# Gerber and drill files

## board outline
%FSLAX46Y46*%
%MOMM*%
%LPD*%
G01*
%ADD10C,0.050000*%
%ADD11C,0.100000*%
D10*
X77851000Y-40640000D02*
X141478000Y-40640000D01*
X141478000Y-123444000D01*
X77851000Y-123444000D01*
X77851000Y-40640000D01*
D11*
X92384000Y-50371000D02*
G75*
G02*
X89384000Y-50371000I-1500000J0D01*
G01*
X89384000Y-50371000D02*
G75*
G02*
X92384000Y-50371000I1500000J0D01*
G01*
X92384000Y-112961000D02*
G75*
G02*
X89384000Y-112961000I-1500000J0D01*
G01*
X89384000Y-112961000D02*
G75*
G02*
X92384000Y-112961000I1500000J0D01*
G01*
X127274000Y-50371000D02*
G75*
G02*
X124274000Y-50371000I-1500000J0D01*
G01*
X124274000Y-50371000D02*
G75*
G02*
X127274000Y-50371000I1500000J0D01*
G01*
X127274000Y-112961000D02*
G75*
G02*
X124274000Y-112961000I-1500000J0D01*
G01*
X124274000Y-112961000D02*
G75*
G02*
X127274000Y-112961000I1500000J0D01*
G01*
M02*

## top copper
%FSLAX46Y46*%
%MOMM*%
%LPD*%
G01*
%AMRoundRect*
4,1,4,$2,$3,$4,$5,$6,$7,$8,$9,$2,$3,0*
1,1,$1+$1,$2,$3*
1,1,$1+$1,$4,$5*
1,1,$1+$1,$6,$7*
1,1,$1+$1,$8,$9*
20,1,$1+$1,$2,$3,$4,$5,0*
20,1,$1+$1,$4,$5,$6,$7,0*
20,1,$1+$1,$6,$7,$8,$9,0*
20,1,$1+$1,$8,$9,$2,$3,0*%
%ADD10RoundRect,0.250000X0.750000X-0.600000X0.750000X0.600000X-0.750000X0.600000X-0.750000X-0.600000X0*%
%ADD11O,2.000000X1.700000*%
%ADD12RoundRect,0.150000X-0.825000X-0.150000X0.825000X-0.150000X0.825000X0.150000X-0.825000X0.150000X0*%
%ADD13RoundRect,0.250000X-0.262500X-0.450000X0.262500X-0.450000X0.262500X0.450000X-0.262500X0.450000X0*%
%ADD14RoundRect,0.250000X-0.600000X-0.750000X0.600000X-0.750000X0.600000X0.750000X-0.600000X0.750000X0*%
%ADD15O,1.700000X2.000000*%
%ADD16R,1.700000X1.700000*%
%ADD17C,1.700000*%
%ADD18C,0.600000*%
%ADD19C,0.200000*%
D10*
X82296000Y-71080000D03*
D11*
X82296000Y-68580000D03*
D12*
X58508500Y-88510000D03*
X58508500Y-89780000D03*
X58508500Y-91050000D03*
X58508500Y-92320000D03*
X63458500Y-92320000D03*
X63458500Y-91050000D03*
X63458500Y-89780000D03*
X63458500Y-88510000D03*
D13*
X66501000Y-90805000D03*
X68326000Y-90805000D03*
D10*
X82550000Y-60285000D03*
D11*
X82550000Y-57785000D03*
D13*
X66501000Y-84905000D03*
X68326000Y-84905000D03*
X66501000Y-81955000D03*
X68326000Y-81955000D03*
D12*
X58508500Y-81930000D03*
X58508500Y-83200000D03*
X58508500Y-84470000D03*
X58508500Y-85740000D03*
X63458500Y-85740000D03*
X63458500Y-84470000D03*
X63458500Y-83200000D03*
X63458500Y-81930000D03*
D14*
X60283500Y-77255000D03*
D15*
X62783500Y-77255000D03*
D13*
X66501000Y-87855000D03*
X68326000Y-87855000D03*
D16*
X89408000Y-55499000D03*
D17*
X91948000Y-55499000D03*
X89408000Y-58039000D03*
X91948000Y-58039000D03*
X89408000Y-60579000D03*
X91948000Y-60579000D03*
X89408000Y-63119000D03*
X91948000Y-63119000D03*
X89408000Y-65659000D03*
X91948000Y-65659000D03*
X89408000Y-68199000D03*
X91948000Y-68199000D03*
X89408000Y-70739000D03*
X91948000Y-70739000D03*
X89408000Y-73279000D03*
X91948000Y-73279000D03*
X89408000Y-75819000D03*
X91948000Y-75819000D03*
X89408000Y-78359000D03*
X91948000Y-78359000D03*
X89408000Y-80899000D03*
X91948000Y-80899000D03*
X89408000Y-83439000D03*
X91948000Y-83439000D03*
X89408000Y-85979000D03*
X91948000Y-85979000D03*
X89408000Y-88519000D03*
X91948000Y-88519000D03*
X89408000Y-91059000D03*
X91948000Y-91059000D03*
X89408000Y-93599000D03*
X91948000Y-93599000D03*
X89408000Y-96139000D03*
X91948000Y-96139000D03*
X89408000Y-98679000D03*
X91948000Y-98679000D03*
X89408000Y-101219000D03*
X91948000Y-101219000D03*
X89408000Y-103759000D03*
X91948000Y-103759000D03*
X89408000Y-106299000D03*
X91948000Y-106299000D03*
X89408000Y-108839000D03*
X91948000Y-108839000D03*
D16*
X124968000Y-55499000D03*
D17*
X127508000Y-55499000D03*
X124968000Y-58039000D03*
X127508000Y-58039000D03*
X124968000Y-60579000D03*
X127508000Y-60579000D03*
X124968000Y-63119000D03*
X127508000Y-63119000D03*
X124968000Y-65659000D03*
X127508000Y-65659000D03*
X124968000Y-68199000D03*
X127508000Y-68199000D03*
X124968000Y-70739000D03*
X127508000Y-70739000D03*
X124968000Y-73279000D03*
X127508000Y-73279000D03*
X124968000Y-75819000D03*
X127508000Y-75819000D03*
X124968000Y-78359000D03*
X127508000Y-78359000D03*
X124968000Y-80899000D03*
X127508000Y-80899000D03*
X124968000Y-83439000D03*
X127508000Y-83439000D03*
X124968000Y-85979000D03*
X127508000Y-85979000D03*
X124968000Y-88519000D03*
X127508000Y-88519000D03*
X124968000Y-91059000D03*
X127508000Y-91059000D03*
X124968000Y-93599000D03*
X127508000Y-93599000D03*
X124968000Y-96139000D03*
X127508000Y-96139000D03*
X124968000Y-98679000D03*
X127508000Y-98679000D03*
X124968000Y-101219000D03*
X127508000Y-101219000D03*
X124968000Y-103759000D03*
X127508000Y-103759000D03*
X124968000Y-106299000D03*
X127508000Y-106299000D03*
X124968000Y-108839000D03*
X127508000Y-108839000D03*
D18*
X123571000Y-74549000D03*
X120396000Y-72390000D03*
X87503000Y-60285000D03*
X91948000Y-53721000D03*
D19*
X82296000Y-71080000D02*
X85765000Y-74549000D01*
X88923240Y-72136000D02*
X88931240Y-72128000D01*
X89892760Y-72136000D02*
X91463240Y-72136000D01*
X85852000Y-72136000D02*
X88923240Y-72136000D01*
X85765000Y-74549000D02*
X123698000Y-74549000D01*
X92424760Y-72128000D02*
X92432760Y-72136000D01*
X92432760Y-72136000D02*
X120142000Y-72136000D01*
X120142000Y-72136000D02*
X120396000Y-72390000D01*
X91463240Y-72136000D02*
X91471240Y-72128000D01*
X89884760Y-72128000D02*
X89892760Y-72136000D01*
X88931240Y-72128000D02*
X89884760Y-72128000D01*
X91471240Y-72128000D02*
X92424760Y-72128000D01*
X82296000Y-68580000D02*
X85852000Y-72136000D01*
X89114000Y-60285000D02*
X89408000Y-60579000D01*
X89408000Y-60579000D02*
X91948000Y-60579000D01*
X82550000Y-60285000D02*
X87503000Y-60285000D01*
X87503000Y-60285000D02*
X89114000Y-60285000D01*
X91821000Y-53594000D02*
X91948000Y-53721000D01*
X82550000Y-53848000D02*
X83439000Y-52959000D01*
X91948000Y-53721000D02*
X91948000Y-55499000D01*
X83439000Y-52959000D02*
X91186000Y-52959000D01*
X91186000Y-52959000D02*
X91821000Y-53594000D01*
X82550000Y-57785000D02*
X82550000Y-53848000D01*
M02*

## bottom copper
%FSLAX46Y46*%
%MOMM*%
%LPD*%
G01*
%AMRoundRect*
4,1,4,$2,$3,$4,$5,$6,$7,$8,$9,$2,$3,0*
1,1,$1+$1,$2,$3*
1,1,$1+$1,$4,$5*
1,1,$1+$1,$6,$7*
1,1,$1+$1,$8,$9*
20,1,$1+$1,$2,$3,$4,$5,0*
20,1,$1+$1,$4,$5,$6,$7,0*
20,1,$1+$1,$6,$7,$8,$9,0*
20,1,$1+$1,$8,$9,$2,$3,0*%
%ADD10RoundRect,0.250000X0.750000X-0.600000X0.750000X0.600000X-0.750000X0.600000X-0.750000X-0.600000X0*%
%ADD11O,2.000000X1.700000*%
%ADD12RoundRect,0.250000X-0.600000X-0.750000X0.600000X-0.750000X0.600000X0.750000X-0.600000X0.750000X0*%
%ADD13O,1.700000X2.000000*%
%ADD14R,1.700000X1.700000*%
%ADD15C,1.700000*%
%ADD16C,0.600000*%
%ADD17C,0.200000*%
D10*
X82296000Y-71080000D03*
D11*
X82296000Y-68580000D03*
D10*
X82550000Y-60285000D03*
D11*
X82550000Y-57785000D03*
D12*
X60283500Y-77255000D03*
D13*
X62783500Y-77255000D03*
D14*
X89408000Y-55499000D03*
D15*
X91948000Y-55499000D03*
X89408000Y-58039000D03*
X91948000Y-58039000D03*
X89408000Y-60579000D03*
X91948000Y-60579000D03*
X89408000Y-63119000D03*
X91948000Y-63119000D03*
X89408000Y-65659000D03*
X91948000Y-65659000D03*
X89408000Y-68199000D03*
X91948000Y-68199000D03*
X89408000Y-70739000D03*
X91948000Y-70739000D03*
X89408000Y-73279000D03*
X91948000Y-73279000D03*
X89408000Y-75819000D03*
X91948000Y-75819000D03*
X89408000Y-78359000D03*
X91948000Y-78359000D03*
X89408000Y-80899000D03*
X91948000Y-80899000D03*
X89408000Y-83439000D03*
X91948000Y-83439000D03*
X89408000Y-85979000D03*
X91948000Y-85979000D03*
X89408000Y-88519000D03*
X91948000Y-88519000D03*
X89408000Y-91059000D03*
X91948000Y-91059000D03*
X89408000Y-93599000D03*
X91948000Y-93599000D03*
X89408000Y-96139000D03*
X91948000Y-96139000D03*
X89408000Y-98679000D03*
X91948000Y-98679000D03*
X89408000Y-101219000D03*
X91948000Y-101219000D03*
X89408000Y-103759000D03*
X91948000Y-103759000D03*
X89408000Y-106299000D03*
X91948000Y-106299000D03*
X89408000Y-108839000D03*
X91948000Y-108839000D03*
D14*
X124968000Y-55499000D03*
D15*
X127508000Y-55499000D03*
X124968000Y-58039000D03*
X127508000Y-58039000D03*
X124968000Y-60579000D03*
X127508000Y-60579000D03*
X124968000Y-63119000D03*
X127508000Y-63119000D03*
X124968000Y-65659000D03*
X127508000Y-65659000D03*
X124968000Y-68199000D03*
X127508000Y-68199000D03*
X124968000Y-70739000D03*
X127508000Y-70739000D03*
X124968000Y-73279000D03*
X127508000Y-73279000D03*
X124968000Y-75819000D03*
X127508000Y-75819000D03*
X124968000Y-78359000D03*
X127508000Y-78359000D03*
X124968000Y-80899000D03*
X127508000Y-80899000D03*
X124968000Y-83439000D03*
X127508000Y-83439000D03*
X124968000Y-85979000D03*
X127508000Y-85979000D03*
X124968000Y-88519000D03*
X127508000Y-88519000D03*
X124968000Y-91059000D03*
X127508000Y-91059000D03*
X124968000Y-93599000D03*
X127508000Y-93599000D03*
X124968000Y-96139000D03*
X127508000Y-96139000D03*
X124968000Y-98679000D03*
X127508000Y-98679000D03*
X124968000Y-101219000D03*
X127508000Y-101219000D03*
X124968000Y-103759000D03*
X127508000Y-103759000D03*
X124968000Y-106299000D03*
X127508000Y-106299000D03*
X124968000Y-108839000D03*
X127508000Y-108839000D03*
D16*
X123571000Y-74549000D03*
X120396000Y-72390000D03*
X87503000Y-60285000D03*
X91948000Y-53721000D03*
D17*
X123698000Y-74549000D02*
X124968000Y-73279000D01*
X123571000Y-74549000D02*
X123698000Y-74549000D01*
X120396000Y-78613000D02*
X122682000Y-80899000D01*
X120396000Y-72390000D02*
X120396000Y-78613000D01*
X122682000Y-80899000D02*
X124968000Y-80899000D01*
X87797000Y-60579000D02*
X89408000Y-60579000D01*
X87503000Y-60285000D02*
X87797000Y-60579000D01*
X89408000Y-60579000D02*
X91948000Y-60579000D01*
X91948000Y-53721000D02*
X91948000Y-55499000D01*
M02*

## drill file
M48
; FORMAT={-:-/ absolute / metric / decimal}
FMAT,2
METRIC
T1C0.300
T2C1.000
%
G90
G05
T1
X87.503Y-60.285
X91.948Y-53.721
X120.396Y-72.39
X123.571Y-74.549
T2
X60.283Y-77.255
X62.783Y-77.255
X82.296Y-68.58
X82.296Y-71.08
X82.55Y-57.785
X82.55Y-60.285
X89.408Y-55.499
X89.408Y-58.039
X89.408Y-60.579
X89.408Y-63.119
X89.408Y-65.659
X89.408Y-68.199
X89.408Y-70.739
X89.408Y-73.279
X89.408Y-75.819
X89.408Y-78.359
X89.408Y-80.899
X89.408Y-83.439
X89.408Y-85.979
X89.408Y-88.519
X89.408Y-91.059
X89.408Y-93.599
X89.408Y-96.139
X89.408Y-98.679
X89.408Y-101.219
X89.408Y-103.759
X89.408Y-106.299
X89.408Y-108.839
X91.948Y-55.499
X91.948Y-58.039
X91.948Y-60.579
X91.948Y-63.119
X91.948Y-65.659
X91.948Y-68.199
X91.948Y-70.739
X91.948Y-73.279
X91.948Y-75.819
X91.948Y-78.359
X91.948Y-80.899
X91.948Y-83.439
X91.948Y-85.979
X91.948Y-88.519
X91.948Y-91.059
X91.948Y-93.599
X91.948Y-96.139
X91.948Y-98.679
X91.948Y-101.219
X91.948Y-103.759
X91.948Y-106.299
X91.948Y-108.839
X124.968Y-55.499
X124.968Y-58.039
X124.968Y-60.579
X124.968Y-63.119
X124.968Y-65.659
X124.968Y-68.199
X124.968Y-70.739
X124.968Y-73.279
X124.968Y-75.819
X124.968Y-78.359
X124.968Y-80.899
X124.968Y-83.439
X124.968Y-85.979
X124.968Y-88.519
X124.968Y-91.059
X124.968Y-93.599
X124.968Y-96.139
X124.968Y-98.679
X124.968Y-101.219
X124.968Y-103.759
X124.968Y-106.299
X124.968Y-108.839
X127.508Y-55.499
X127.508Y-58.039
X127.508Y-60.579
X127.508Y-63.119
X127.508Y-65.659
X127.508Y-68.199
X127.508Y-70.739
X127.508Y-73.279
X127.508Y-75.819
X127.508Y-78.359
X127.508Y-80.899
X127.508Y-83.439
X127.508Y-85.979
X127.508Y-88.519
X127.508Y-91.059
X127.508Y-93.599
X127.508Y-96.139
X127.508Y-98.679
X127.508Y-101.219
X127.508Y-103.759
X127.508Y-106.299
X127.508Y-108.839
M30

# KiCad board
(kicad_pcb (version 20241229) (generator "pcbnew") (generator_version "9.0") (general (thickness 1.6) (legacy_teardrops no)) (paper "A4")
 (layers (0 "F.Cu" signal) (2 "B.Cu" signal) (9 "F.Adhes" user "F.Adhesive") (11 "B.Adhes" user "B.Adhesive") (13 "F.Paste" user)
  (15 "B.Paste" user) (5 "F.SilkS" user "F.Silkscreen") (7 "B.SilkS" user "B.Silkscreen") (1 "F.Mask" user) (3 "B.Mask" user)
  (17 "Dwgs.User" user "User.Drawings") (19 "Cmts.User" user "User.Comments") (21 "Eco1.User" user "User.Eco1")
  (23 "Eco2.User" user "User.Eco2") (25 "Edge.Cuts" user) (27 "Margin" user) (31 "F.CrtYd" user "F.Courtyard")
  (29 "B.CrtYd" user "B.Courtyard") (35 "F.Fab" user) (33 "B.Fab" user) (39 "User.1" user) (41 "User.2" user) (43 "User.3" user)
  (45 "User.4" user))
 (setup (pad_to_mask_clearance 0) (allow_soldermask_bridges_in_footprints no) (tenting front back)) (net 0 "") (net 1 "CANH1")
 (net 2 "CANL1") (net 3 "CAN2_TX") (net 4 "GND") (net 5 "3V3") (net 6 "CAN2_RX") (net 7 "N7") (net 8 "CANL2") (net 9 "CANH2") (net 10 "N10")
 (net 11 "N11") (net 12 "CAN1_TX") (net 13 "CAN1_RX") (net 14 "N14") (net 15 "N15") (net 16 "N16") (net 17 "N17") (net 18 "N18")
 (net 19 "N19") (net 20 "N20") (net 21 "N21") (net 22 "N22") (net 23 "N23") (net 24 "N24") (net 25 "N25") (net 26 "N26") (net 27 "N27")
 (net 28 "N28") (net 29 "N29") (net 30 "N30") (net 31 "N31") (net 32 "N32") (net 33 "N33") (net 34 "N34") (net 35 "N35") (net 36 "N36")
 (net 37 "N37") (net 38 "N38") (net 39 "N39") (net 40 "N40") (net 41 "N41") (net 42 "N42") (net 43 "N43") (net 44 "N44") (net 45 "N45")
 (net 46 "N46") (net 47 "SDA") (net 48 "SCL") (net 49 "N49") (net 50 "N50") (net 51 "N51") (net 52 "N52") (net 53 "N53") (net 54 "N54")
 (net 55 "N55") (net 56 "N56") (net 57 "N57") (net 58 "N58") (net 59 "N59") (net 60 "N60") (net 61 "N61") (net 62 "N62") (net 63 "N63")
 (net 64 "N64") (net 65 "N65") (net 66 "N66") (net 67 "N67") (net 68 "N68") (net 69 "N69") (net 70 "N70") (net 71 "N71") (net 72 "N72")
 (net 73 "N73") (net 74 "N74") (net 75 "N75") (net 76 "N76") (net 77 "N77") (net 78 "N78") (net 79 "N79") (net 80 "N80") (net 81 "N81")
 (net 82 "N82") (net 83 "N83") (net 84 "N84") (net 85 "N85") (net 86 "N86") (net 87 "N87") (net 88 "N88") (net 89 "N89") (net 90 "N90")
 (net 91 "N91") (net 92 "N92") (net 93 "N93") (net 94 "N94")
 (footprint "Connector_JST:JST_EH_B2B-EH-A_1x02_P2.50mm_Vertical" (layer "F.Cu") (at 82.296 71.08 90)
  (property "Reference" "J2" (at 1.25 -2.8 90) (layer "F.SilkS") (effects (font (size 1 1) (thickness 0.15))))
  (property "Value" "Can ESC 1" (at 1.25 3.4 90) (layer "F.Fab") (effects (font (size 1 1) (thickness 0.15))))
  (pad "1" thru_hole roundrect (at 0 0 90) (size 1.7 2) (drill 1) (layers "*.Cu" "*.Mask") (remove_unused_layers no)
   (roundrect_rratio 0.147059) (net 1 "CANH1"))
  (pad "2" thru_hole oval (at 2.5 0 90) (size 1.7 2) (drill 1) (layers "*.Cu" "*.Mask") (remove_unused_layers no) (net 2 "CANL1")))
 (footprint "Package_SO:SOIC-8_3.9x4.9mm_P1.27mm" (layer "F.Cu") (at 60.9835 90.415)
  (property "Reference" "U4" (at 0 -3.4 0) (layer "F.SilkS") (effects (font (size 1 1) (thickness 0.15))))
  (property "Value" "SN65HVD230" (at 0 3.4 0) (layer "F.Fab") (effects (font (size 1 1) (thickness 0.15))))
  (pad "1" smd roundrect (at -2.475 -1.905) (size 1.95 0.6) (layers "F.Cu" "F.Mask" "F.Paste") (roundrect_rratio 0.25) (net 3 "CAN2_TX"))
  (pad "2" smd roundrect (at -2.475 -0.635) (size 1.95 0.6) (layers "F.Cu" "F.Mask" "F.Paste") (roundrect_rratio 0.25) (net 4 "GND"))
  (pad "3" smd roundrect (at -2.475 0.635) (size 1.95 0.6) (layers "F.Cu" "F.Mask" "F.Paste") (roundrect_rratio 0.25) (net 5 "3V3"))
  (pad "4" smd roundrect (at -2.475 1.905) (size 1.95 0.6) (layers "F.Cu" "F.Mask" "F.Paste") (roundrect_rratio 0.25) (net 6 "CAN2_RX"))
  (pad "5" smd roundrect (at 2.475 1.905) (size 1.95 0.6) (layers "F.Cu" "F.Mask" "F.Paste") (roundrect_rratio 0.25) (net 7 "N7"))
  (pad "6" smd roundrect (at 2.475 0.635) (size 1.95 0.6) (layers "F.Cu" "F.Mask" "F.Paste") (roundrect_rratio 0.25) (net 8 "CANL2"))
  (pad "7" smd roundrect (at 2.475 -0.635) (size 1.95 0.6) (layers "F.Cu" "F.Mask" "F.Paste") (roundrect_rratio 0.25) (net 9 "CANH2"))
  (pad "8" smd roundrect (at 2.475 -1.905) (size 1.95 0.6) (layers "F.Cu" "F.Mask" "F.Paste") (roundrect_rratio 0.25) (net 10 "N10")))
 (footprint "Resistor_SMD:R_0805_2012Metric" (layer "F.Cu") (at 67.4135 90.805)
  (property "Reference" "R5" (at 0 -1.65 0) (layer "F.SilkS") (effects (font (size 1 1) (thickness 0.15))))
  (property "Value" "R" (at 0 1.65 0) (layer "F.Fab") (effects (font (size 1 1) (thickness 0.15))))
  (pad "1" smd roundrect (at -0.9125 0) (size 1.025 1.4) (layers "F.Cu" "F.Mask" "F.Paste") (roundrect_rratio 0.243902) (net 4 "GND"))
  (pad "2" smd roundrect (at 0.9125 0) (size 1.025 1.4) (layers "F.Cu" "F.Mask" "F.Paste") (roundrect_rratio 0.243902) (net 10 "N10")))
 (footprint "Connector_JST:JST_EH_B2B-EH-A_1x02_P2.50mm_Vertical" (layer "F.Cu") (at 82.55 60.285 90)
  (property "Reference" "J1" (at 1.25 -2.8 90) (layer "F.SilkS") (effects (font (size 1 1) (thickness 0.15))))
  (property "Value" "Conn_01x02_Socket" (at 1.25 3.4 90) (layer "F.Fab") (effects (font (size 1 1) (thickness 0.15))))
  (pad "1" thru_hole roundrect (at 0 0 90) (size 1.7 2) (drill 1) (layers "*.Cu" "*.Mask") (remove_unused_layers no)
   (roundrect_rratio 0.147059) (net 4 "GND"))
  (pad "2" thru_hole oval (at 2.5 0 90) (size 1.7 2) (drill 1) (layers "*.Cu" "*.Mask") (remove_unused_layers no) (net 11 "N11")))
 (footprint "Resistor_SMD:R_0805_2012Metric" (layer "F.Cu") (at 67.4135 84.905)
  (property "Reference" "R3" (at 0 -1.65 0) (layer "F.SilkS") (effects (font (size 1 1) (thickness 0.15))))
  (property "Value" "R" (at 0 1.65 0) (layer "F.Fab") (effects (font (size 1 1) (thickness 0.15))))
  (pad "1" smd roundrect (at -0.9125 0) (size 1.025 1.4) (layers "F.Cu" "F.Mask" "F.Paste") (roundrect_rratio 0.243902) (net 9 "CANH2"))
  (pad "2" smd roundrect (at 0.9125 0) (size 1.025 1.4) (layers "F.Cu" "F.Mask" "F.Paste") (roundrect_rratio 0.243902) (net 8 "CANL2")))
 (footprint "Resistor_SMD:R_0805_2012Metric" (layer "F.Cu") (at 67.4135 81.955)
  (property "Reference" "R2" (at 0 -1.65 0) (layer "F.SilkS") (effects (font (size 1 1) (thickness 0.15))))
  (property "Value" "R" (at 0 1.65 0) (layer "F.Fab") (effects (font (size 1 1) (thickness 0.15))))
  (pad "1" smd roundrect (at -0.9125 0) (size 1.025 1.4) (layers "F.Cu" "F.Mask" "F.Paste") (roundrect_rratio 0.243902) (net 1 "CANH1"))
  (pad "2" smd roundrect (at 0.9125 0) (size 1.025 1.4) (layers "F.Cu" "F.Mask" "F.Paste") (roundrect_rratio 0.243902) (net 2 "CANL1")))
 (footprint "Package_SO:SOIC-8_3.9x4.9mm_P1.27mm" (layer "F.Cu") (at 60.9835 83.835)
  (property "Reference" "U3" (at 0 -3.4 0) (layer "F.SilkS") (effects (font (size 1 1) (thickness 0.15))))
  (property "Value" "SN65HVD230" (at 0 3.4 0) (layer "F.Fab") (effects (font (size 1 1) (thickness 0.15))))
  (pad "1" smd roundrect (at -2.475 -1.905) (size 1.95 0.6) (layers "F.Cu" "F.Mask" "F.Paste") (roundrect_rratio 0.25) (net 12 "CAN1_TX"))
  (pad "2" smd roundrect (at -2.475 -0.635) (size 1.95 0.6) (layers "F.Cu" "F.Mask" "F.Paste") (roundrect_rratio 0.25) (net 4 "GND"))
  (pad "3" smd roundrect (at -2.475 0.635) (size 1.95 0.6) (layers "F.Cu" "F.Mask" "F.Paste") (roundrect_rratio 0.25) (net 5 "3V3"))
  (pad "4" smd roundrect (at -2.475 1.905) (size 1.95 0.6) (layers "F.Cu" "F.Mask" "F.Paste") (roundrect_rratio 0.25) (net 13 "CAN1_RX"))
  (pad "5" smd roundrect (at 2.475 1.905) (size 1.95 0.6) (layers "F.Cu" "F.Mask" "F.Paste") (roundrect_rratio 0.25) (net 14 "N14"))
  (pad "6" smd roundrect (at 2.475 0.635) (size 1.95 0.6) (layers "F.Cu" "F.Mask" "F.Paste") (roundrect_rratio 0.25) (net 2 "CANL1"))
  (pad "7" smd roundrect (at 2.475 -0.635) (size 1.95 0.6) (layers "F.Cu" "F.Mask" "F.Paste") (roundrect_rratio 0.25) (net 1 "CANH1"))
  (pad "8" smd roundrect (at 2.475 -1.905) (size 1.95 0.6) (layers "F.Cu" "F.Mask" "F.Paste") (roundrect_rratio 0.25) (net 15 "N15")))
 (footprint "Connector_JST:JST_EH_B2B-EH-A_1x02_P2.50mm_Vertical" (layer "F.Cu") (at 60.2835 77.255)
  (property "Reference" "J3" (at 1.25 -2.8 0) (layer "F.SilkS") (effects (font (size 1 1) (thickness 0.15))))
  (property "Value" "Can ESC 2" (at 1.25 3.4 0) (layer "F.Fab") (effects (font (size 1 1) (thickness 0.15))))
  (pad "1" thru_hole roundrect (at 0 0) (size 1.7 2) (drill 1) (layers "*.Cu" "*.Mask") (remove_unused_layers no)
   (roundrect_rratio 0.147059) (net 9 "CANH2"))
  (pad "2" thru_hole oval (at 2.5 0) (size 1.7 2) (drill 1) (layers "*.Cu" "*.Mask") (remove_unused_layers no) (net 8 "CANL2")))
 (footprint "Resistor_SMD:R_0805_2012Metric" (layer "F.Cu") (at 67.4135 87.855)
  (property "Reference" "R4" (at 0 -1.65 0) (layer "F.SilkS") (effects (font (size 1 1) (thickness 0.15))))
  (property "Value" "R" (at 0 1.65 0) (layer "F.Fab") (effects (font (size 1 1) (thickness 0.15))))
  (pad "1" smd roundrect (at -0.9125 0) (size 1.025 1.4) (layers "F.Cu" "F.Mask" "F.Paste") (roundrect_rratio 0.243902) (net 4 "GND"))
  (pad "2" smd roundrect (at 0.9125 0) (size 1.025 1.4) (layers "F.Cu" "F.Mask" "F.Paste") (roundrect_rratio 0.243902) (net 15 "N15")))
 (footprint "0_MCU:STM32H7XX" (layer "F.Cu") (at 99.568 38.735)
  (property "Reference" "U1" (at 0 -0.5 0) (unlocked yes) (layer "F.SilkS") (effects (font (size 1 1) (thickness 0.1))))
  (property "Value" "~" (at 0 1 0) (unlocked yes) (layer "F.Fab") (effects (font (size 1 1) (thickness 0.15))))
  (fp_circle (center -8.684 11.636) (end -7.184 11.636) (stroke (width 0.1) (type solid)) (fill no) (layer "Edge.Cuts"))
  (fp_circle (center -8.684 74.226) (end -7.184 74.226) (stroke (width 0.1) (type solid)) (fill no) (layer "Edge.Cuts"))
  (fp_circle (center 26.206 11.636) (end 27.706 11.636) (stroke (width 0.1) (type solid)) (fill no) (layer "Edge.Cuts"))
  (fp_circle (center 26.206 74.226) (end 27.706 74.226) (stroke (width 0.1) (type solid)) (fill no) (layer "Edge.Cuts"))
  (pad "1" thru_hole rect (at -10.16 16.764 180) (size 1.7 1.7) (drill 1) (layers "*.Cu" "*.Mask") (remove_unused_layers no) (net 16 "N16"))
  (pad "2" thru_hole circle (at -7.62 16.764 180) (size 1.7 1.7) (drill 1) (layers "*.Cu" "*.Mask") (remove_unused_layers no) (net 11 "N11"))
  (pad "3" thru_hole circle (at -10.16 19.304 180) (size 1.7 1.7) (drill 1) (layers "*.Cu" "*.Mask") (remove_unused_layers no) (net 5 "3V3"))
  (pad "4" thru_hole circle (at -7.62 19.304 180) (size 1.7 1.7) (drill 1) (layers "*.Cu" "*.Mask") (remove_unused_layers no) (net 5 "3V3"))
  (pad "5" thru_hole circle (at -10.16 21.844 180) (size 1.7 1.7) (drill 1) (layers "*.Cu" "*.Mask") (remove_unused_layers no) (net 4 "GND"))
  (pad "6" thru_hole circle (at -7.62 21.844 180) (size 1.7 1.7) (drill 1) (layers "*.Cu" "*.Mask") (remove_unused_layers no) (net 4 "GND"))
  (pad "7" thru_hole circle (at -10.16 24.384 180) (size 1.7 1.7) (drill 1) (layers "*.Cu" "*.Mask") (remove_unused_layers no)
   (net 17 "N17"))
  (pad "8" thru_hole circle (at -7.62 24.384 180) (size 1.7 1.7) (drill 1) (layers "*.Cu" "*.Mask") (remove_unused_layers no) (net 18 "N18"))
  (pad "9" thru_hole circle (at -10.16 26.924 180) (size 1.7 1.7) (drill 1) (layers "*.Cu" "*.Mask") (remove_unused_layers no)
   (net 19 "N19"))
  (pad "10" thru_hole circle (at -7.62 26.924 180) (size 1.7 1.7) (drill 1) (layers "*.Cu" "*.Mask") (remove_unused_layers no)
   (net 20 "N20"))
  (pad "11" thru_hole circle (at -10.16 29.464 180) (size 1.7 1.7) (drill 1) (layers "*.Cu" "*.Mask") (remove_unused_layers no)
   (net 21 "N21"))
  (pad "12" thru_hole circle (at -7.62 29.464 180) (size 1.7 1.7) (drill 1) (layers "*.Cu" "*.Mask") (remove_unused_layers no)
   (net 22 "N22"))
  (pad "13" thru_hole circle (at -10.16 32.004 180) (size 1.7 1.7) (drill 1) (layers "*.Cu" "*.Mask") (remove_unused_layers no)
   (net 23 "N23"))
  (pad "14" thru_hole circle (at -7.62 32.004 180) (size 1.7 1.7) (drill 1) (layers "*.Cu" "*.Mask") (remove_unused_layers no)
   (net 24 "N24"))
  (pad "15" thru_hole circle (at -10.16 34.544 180) (size 1.7 1.7) (drill 1) (layers "*.Cu" "*.Mask") (remove_unused_layers no)
   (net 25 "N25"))
  (pad "16" thru_hole circle (at -7.62 34.544 180) (size 1.7 1.7) (drill 1) (layers "*.Cu" "*.Mask") (remove_unused_layers no)
   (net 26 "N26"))
  (pad "17" thru_hole circle (at -10.16 37.084 180) (size 1.7 1.7) (drill 1) (layers "*.Cu" "*.Mask") (remove_unused_layers no)
   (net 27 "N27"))
  (pad "18" thru_hole circle (at -7.62 37.084 180) (size 1.7 1.7) (drill 1) (layers "*.Cu" "*.Mask") (remove_unused_layers no)
   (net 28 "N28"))
  (pad "19" thru_hole circle (at -10.16 39.624 180) (size 1.7 1.7) (drill 1) (layers "*.Cu" "*.Mask") (remove_unused_layers no)
   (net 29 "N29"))
  (pad "20" thru_hole circle (at -7.62 39.624 180) (size 1.7 1.7) (drill 1) (layers "*.Cu" "*.Mask") (remove_unused_layers no)
   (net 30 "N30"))
  (pad "21" thru_hole circle (at -10.16 42.164 180) (size 1.7 1.7) (drill 1) (layers "*.Cu" "*.Mask") (remove_unused_layers no)
   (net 12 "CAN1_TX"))
  (pad "22" thru_hole circle (at -7.62 42.164 180) (size 1.7 1.7) (drill 1) (layers "*.Cu" "*.Mask") (remove_unused_layers no)
   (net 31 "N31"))
  (pad "23" thru_hole circle (at -10.16 44.704 180) (size 1.7 1.7) (drill 1) (layers "*.Cu" "*.Mask") (remove_unused_layers no)
   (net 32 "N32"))
  (pad "24" thru_hole circle (at -7.62 44.704 180) (size 1.7 1.7) (drill 1) (layers "*.Cu" "*.Mask") (remove_unused_layers no)
   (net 13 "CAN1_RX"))
  (pad "25" thru_hole circle (at -10.16 47.244 180) (size 1.7 1.7) (drill 1) (layers "*.Cu" "*.Mask") (remove_unused_layers no)
   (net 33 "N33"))
  (pad "26" thru_hole circle (at -7.62 47.244 180) (size 1.7 1.7) (drill 1) (layers "*.Cu" "*.Mask") (remove_unused_layers no)
   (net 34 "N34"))
  (pad "27" thru_hole circle (at -10.16 49.784 180) (size 1.7 1.7) (drill 1) (layers "*.Cu" "*.Mask") (remove_unused_layers no)
   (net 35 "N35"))
  (pad "28" thru_hole circle (at -7.62 49.784 180) (size 1.7 1.7) (drill 1) (layers "*.Cu" "*.Mask") (remove_unused_layers no)
   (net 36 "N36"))
  (pad "29" thru_hole circle (at -10.16 52.324 180) (size 1.7 1.7) (drill 1) (layers "*.Cu" "*.Mask") (remove_unused_layers no)
   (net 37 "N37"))
  (pad "30" thru_hole circle (at -7.62 52.324 180) (size 1.7 1.7) (drill 1) (layers "*.Cu" "*.Mask") (remove_unused_layers no)
   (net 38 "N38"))
  (pad "31" thru_hole circle (at -10.16 54.864 180) (size 1.7 1.7) (drill 1) (layers "*.Cu" "*.Mask") (remove_unused_layers no)
   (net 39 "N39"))
  (pad "32" thru_hole circle (at -7.62 54.864 180) (size 1.7 1.7) (drill 1) (layers "*.Cu" "*.Mask") (remove_unused_layers no)
   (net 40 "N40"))
  (pad "33" thru_hole circle (at -10.16 57.404 180) (size 1.7 1.7) (drill 1) (layers "*.Cu" "*.Mask") (remove_unused_layers no)
   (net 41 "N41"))
  (pad "34" thru_hole circle (at -7.62 57.404 180) (size 1.7 1.7) (drill 1) (layers "*.Cu" "*.Mask") (remove_unused_layers no)
   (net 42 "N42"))
  (pad "35" thru_hole circle (at -10.16 59.944 180) (size 1.7 1.7) (drill 1) (layers "*.Cu" "*.Mask") (remove_unused_layers no)
   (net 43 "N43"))
  (pad "36" thru_hole circle (at -7.62 59.944 180) (size 1.7 1.7) (drill 1) (layers "*.Cu" "*.Mask") (remove_unused_layers no)
   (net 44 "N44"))
  (pad "37" thru_hole circle (at -10.16 62.484 180) (size 1.7 1.7) (drill 1) (layers "*.Cu" "*.Mask") (remove_unused_layers no)
   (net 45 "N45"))
  (pad "38" thru_hole circle (at -7.62 62.484 180) (size 1.7 1.7) (drill 1) (layers "*.Cu" "*.Mask") (remove_unused_layers no)
   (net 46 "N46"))
  (pad "39" thru_hole circle (at -10.16 65.024 180) (size 1.7 1.7) (drill 1) (layers "*.Cu" "*.Mask") (remove_unused_layers no)
   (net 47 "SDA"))
  (pad "40" thru_hole circle (at -7.62 65.024 180) (size 1.7 1.7) (drill 1) (layers "*.Cu" "*.Mask") (remove_unused_layers no)
   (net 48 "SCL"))
  (pad "41" thru_hole circle (at -10.16 67.564 180) (size 1.7 1.7) (drill 1) (layers "*.Cu" "*.Mask") (remove_unused_layers no)
   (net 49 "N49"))
  (pad "42" thru_hole circle (at -7.62 67.564 180) (size 1.7 1.7) (drill 1) (layers "*.Cu" "*.Mask") (remove_unused_layers no)
   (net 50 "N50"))
  (pad "43" thru_hole circle (at -10.16 70.104 180) (size 1.7 1.7) (drill 1) (layers "*.Cu" "*.Mask") (remove_unused_layers no)
   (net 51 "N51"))
  (pad "44" thru_hole circle (at -7.62 70.104 180) (size 1.7 1.7) (drill 1) (layers "*.Cu" "*.Mask") (remove_unused_layers no)
   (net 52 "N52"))
  (pad "45" thru_hole rect (at 25.4 16.764 180) (size 1.7 1.7) (drill 1) (layers "*.Cu" "*.Mask") (remove_unused_layers no) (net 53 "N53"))
  (pad "46" thru_hole circle (at 27.94 16.764 180) (size 1.7 1.7) (drill 1) (layers "*.Cu" "*.Mask") (remove_unused_layers no)
   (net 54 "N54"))
  (pad "47" thru_hole circle (at 25.4 19.304 180) (size 1.7 1.7) (drill 1) (layers "*.Cu" "*.Mask") (remove_unused_layers no) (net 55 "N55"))
  (pad "48" thru_hole circle (at 27.94 19.304 180) (size 1.7 1.7) (drill 1) (layers "*.Cu" "*.Mask") (remove_unused_layers no)
   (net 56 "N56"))
  (pad "49" thru_hole circle (at 25.4 21.844 180) (size 1.7 1.7) (drill 1) (layers "*.Cu" "*.Mask") (remove_unused_layers no) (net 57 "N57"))
  (pad "50" thru_hole circle (at 27.94 21.844 180) (size 1.7 1.7) (drill 1) (layers "*.Cu" "*.Mask") (remove_unused_layers no)
   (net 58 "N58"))
  (pad "51" thru_hole circle (at 25.4 24.384 180) (size 1.7 1.7) (drill 1) (layers "*.Cu" "*.Mask") (remove_unused_layers no) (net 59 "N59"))
  (pad "52" thru_hole circle (at 27.94 24.384 180) (size 1.7 1.7) (drill 1) (layers "*.Cu" "*.Mask") (remove_unused_layers no)
   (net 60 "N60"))
  (pad "53" thru_hole circle (at 25.4 26.924 180) (size 1.7 1.7) (drill 1) (layers "*.Cu" "*.Mask") (remove_unused_layers no)
   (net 6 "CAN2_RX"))
  (pad "54" thru_hole circle (at 27.94 26.924 180) (size 1.7 1.7) (drill 1) (layers "*.Cu" "*.Mask") (remove_unused_layers no)
   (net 3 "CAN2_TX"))
  (pad "55" thru_hole circle (at 25.4 29.464 180) (size 1.7 1.7) (drill 1) (layers "*.Cu" "*.Mask") (remove_unused_layers no) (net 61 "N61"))
  (pad "56" thru_hole circle (at 27.94 29.464 180) (size 1.7 1.7) (drill 1) (layers "*.Cu" "*.Mask") (remove_unused_layers no)
   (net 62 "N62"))
  (pad "57" thru_hole circle (at 25.4 32.004 180) (size 1.7 1.7) (drill 1) (layers "*.Cu" "*.Mask") (remove_unused_layers no) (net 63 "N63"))
  (pad "58" thru_hole circle (at 27.94 32.004 180) (size 1.7 1.7) (drill 1) (layers "*.Cu" "*.Mask") (remove_unused_layers no)
   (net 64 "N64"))
  (pad "59" thru_hole circle (at 25.4 34.544 180) (size 1.7 1.7) (drill 1) (layers "*.Cu" "*.Mask") (remove_unused_layers no) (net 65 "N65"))
  (pad "60" thru_hole circle (at 27.94 34.544 180) (size 1.7 1.7) (drill 1) (layers "*.Cu" "*.Mask") (remove_unused_layers no)
   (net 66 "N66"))
  (pad "61" thru_hole circle (at 25.4 37.084 180) (size 1.7 1.7) (drill 1) (layers "*.Cu" "*.Mask") (remove_unused_layers no) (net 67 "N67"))
  (pad "62" thru_hole circle (at 27.94 37.084 180) (size 1.7 1.7) (drill 1) (layers "*.Cu" "*.Mask") (remove_unused_layers no)
   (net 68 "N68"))
  (pad "63" thru_hole circle (at 25.4 39.624 180) (size 1.7 1.7) (drill 1) (layers "*.Cu" "*.Mask") (remove_unused_layers no) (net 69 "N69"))
  (pad "64" thru_hole circle (at 27.94 39.624 180) (size 1.7 1.7) (drill 1) (layers "*.Cu" "*.Mask") (remove_unused_layers no)
   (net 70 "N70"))
  (pad "65" thru_hole circle (at 25.4 42.164 180) (size 1.7 1.7) (drill 1) (layers "*.Cu" "*.Mask") (remove_unused_layers no) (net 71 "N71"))
  (pad "66" thru_hole circle (at 27.94 42.164 180) (size 1.7 1.7) (drill 1) (layers "*.Cu" "*.Mask") (remove_unused_layers no)
   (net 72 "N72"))
  (pad "67" thru_hole circle (at 25.4 44.704 180) (size 1.7 1.7) (drill 1) (layers "*.Cu" "*.Mask") (remove_unused_layers no) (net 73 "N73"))
  (pad "68" thru_hole circle (at 27.94 44.704 180) (size 1.7 1.7) (drill 1) (layers "*.Cu" "*.Mask") (remove_unused_layers no)
   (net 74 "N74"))
  (pad "69" thru_hole circle (at 25.4 47.244 180) (size 1.7 1.7) (drill 1) (layers "*.Cu" "*.Mask") (remove_unused_layers no) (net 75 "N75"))
  (pad "70" thru_hole circle (at 27.94 47.244 180) (size 1.7 1.7) (drill 1) (layers "*.Cu" "*.Mask") (remove_unused_layers no)
   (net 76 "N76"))
  (pad "71" thru_hole circle (at 25.4 49.784 180) (size 1.7 1.7) (drill 1) (layers "*.Cu" "*.Mask") (remove_unused_layers no) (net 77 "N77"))
  (pad "72" thru_hole circle (at 27.94 49.784 180) (size 1.7 1.7) (drill 1) (layers "*.Cu" "*.Mask") (remove_unused_layers no)
   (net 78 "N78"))
  (pad "73" thru_hole circle (at 25.4 52.324 180) (size 1.7 1.7) (drill 1) (layers "*.Cu" "*.Mask") (remove_unused_layers no) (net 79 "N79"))
  (pad "74" thru_hole circle (at 27.94 52.324 180) (size 1.7 1.7) (drill 1) (layers "*.Cu" "*.Mask") (remove_unused_layers no)
   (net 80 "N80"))
  (pad "75" thru_hole circle (at 25.4 54.864 180) (size 1.7 1.7) (drill 1) (layers "*.Cu" "*.Mask") (remove_unused_layers no) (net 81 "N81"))
  (pad "76" thru_hole circle (at 27.94 54.864 180) (size 1.7 1.7) (drill 1) (layers "*.Cu" "*.Mask") (remove_unused_layers no)
   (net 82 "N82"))
  (pad "77" thru_hole circle (at 25.4 57.404 180) (size 1.7 1.7) (drill 1) (layers "*.Cu" "*.Mask") (remove_unused_layers no) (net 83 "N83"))
  (pad "78" thru_hole circle (at 27.94 57.404 180) (size 1.7 1.7) (drill 1) (layers "*.Cu" "*.Mask") (remove_unused_layers no)
   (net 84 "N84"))
  (pad "79" thru_hole circle (at 25.4 59.944 180) (size 1.7 1.7) (drill 1) (layers "*.Cu" "*.Mask") (remove_unused_layers no) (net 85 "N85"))
  (pad "80" thru_hole circle (at 27.94 59.944 180) (size 1.7 1.7) (drill 1) (layers "*.Cu" "*.Mask") (remove_unused_layers no)
   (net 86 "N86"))
  (pad "81" thru_hole circle (at 25.4 62.484 180) (size 1.7 1.7) (drill 1) (layers "*.Cu" "*.Mask") (remove_unused_layers no) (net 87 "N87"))
  (pad "82" thru_hole circle (at 27.94 62.484 180) (size 1.7 1.7) (drill 1) (layers "*.Cu" "*.Mask") (remove_unused_layers no)
   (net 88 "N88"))
  (pad "83" thru_hole circle (at 25.4 65.024 180) (size 1.7 1.7) (drill 1) (layers "*.Cu" "*.Mask") (remove_unused_layers no) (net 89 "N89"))
  (pad "84" thru_hole circle (at 27.94 65.024 180) (size 1.7 1.7) (drill 1) (layers "*.Cu" "*.Mask") (remove_unused_layers no)
   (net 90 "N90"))
  (pad "85" thru_hole circle (at 25.4 67.564 180) (size 1.7 1.7) (drill 1) (layers "*.Cu" "*.Mask") (remove_unused_layers no) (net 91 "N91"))
  (pad "86" thru_hole circle (at 27.94 67.564 180) (size 1.7 1.7) (drill 1) (layers "*.Cu" "*.Mask") (remove_unused_layers no)
   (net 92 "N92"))
  (pad "87" thru_hole circle (at 25.4 70.104 180) (size 1.7 1.7) (drill 1) (layers "*.Cu" "*.Mask") (remove_unused_layers no) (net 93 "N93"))
  (pad "88" thru_hole circle (at 27.94 70.104 180) (size 1.7 1.7) (drill 1) (layers "*.Cu" "*.Mask") (remove_unused_layers no)
   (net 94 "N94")))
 (gr_rect (start 77.851 40.64) (end 141.478 123.444) (stroke (width 0.05) (type default)) (fill no) (layer "Edge.Cuts"))
 (segment (start 82.296 71.08) (end 85.765 74.549) (width 0.2) (layer "F.Cu") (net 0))
 (segment (start 88.92324 72.136) (end 88.93124 72.128) (width 0.2) (layer "F.Cu") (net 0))
 (segment (start 89.89276 72.136) (end 91.46324 72.136) (width 0.2) (layer "F.Cu") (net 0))
 (segment (start 85.852 72.136) (end 88.92324 72.136) (width 0.2) (layer "F.Cu") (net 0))
 (segment (start 85.765 74.549) (end 123.698 74.549) (width 0.2) (layer "F.Cu") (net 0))
 (segment (start 92.42476 72.128) (end 92.43276 72.136) (width 0.2) (layer "F.Cu") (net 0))
 (segment (start 92.43276 72.136) (end 120.142 72.136) (width 0.2) (layer "F.Cu") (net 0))
 (segment (start 120.142 72.136) (end 120.396 72.39) (width 0.2) (layer "F.Cu") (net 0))
 (segment (start 91.46324 72.136) (end 91.47124 72.128) (width 0.2) (layer "F.Cu") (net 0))
 (segment (start 89.88476 72.128) (end 89.89276 72.136) (width 0.2) (layer "F.Cu") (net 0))
 (segment (start 88.93124 72.128) (end 89.88476 72.128) (width 0.2) (layer "F.Cu") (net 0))
 (segment (start 91.47124 72.128) (end 92.42476 72.128) (width 0.2) (layer "F.Cu") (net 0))
 (segment (start 82.296 68.58) (end 85.852 72.136) (width 0.2) (layer "F.Cu") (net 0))
 (via (at 123.571 74.549) (size 0.6) (drill 0.3) (layers "F.Cu" "B.Cu") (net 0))
 (via (at 120.396 72.39) (size 0.6) (drill 0.3) (layers "F.Cu" "B.Cu") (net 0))
 (segment (start 123.698 74.549) (end 124.968 73.279) (width 0.2) (layer "B.Cu") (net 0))
 (segment (start 123.571 74.549) (end 123.698 74.549) (width 0.2) (layer "B.Cu") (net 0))
 (segment (start 120.396 78.613) (end 122.682 80.899) (width 0.2) (layer "B.Cu") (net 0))
 (segment (start 120.396 72.39) (end 120.396 78.613) (width 0.2) (layer "B.Cu") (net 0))
 (segment (start 122.682 80.899) (end 124.968 80.899) (width 0.2) (layer "B.Cu") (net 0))
 (segment (start 89.114 60.285) (end 89.408 60.579) (width 0.2) (layer "F.Cu") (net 4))
 (segment (start 89.408 60.579) (end 91.948 60.579) (width 0.2) (layer "F.Cu") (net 4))
 (segment (start 82.55 60.285) (end 87.503 60.285) (width 0.2) (layer "F.Cu") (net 4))
 (segment (start 87.503 60.285) (end 89.114 60.285) (width 0.2) (layer "F.Cu") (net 4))
 (via (at 87.503 60.285) (size 0.6) (drill 0.3) (layers "F.Cu" "B.Cu") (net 4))
 (segment (start 87.797 60.579) (end 89.408 60.579) (width 0.2) (layer "B.Cu") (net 4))
 (segment (start 87.503 60.285) (end 87.797 60.579) (width 0.2) (layer "B.Cu") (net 4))
 (segment (start 89.408 60.579) (end 91.948 60.579) (width 0.2) (layer "B.Cu") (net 4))
 (segment (start 91.821 53.594) (end 91.948 53.721) (width 0.2) (layer "F.Cu") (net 11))
 (segment (start 82.55 53.848) (end 83.439 52.959) (width 0.2) (layer "F.Cu") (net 11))
 (segment (start 91.948 53.721) (end 91.948 55.499) (width 0.2) (layer "F.Cu") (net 11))
 (segment (start 83.439 52.959) (end 91.186 52.959) (width 0.2) (layer "F.Cu") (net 11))
 (segment (start 91.186 52.959) (end 91.821 53.594) (width 0.2) (layer "F.Cu") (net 11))
 (segment (start 82.55 57.785) (end 82.55 53.848) (width 0.2) (layer "F.Cu") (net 11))
 (via (at 91.948 53.721) (size 0.6) (drill 0.3) (layers "F.Cu" "B.Cu") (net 11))
 (segment (start 91.948 53.721) (end 91.948 55.499) (width 0.2) (layer "B.Cu") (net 11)))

